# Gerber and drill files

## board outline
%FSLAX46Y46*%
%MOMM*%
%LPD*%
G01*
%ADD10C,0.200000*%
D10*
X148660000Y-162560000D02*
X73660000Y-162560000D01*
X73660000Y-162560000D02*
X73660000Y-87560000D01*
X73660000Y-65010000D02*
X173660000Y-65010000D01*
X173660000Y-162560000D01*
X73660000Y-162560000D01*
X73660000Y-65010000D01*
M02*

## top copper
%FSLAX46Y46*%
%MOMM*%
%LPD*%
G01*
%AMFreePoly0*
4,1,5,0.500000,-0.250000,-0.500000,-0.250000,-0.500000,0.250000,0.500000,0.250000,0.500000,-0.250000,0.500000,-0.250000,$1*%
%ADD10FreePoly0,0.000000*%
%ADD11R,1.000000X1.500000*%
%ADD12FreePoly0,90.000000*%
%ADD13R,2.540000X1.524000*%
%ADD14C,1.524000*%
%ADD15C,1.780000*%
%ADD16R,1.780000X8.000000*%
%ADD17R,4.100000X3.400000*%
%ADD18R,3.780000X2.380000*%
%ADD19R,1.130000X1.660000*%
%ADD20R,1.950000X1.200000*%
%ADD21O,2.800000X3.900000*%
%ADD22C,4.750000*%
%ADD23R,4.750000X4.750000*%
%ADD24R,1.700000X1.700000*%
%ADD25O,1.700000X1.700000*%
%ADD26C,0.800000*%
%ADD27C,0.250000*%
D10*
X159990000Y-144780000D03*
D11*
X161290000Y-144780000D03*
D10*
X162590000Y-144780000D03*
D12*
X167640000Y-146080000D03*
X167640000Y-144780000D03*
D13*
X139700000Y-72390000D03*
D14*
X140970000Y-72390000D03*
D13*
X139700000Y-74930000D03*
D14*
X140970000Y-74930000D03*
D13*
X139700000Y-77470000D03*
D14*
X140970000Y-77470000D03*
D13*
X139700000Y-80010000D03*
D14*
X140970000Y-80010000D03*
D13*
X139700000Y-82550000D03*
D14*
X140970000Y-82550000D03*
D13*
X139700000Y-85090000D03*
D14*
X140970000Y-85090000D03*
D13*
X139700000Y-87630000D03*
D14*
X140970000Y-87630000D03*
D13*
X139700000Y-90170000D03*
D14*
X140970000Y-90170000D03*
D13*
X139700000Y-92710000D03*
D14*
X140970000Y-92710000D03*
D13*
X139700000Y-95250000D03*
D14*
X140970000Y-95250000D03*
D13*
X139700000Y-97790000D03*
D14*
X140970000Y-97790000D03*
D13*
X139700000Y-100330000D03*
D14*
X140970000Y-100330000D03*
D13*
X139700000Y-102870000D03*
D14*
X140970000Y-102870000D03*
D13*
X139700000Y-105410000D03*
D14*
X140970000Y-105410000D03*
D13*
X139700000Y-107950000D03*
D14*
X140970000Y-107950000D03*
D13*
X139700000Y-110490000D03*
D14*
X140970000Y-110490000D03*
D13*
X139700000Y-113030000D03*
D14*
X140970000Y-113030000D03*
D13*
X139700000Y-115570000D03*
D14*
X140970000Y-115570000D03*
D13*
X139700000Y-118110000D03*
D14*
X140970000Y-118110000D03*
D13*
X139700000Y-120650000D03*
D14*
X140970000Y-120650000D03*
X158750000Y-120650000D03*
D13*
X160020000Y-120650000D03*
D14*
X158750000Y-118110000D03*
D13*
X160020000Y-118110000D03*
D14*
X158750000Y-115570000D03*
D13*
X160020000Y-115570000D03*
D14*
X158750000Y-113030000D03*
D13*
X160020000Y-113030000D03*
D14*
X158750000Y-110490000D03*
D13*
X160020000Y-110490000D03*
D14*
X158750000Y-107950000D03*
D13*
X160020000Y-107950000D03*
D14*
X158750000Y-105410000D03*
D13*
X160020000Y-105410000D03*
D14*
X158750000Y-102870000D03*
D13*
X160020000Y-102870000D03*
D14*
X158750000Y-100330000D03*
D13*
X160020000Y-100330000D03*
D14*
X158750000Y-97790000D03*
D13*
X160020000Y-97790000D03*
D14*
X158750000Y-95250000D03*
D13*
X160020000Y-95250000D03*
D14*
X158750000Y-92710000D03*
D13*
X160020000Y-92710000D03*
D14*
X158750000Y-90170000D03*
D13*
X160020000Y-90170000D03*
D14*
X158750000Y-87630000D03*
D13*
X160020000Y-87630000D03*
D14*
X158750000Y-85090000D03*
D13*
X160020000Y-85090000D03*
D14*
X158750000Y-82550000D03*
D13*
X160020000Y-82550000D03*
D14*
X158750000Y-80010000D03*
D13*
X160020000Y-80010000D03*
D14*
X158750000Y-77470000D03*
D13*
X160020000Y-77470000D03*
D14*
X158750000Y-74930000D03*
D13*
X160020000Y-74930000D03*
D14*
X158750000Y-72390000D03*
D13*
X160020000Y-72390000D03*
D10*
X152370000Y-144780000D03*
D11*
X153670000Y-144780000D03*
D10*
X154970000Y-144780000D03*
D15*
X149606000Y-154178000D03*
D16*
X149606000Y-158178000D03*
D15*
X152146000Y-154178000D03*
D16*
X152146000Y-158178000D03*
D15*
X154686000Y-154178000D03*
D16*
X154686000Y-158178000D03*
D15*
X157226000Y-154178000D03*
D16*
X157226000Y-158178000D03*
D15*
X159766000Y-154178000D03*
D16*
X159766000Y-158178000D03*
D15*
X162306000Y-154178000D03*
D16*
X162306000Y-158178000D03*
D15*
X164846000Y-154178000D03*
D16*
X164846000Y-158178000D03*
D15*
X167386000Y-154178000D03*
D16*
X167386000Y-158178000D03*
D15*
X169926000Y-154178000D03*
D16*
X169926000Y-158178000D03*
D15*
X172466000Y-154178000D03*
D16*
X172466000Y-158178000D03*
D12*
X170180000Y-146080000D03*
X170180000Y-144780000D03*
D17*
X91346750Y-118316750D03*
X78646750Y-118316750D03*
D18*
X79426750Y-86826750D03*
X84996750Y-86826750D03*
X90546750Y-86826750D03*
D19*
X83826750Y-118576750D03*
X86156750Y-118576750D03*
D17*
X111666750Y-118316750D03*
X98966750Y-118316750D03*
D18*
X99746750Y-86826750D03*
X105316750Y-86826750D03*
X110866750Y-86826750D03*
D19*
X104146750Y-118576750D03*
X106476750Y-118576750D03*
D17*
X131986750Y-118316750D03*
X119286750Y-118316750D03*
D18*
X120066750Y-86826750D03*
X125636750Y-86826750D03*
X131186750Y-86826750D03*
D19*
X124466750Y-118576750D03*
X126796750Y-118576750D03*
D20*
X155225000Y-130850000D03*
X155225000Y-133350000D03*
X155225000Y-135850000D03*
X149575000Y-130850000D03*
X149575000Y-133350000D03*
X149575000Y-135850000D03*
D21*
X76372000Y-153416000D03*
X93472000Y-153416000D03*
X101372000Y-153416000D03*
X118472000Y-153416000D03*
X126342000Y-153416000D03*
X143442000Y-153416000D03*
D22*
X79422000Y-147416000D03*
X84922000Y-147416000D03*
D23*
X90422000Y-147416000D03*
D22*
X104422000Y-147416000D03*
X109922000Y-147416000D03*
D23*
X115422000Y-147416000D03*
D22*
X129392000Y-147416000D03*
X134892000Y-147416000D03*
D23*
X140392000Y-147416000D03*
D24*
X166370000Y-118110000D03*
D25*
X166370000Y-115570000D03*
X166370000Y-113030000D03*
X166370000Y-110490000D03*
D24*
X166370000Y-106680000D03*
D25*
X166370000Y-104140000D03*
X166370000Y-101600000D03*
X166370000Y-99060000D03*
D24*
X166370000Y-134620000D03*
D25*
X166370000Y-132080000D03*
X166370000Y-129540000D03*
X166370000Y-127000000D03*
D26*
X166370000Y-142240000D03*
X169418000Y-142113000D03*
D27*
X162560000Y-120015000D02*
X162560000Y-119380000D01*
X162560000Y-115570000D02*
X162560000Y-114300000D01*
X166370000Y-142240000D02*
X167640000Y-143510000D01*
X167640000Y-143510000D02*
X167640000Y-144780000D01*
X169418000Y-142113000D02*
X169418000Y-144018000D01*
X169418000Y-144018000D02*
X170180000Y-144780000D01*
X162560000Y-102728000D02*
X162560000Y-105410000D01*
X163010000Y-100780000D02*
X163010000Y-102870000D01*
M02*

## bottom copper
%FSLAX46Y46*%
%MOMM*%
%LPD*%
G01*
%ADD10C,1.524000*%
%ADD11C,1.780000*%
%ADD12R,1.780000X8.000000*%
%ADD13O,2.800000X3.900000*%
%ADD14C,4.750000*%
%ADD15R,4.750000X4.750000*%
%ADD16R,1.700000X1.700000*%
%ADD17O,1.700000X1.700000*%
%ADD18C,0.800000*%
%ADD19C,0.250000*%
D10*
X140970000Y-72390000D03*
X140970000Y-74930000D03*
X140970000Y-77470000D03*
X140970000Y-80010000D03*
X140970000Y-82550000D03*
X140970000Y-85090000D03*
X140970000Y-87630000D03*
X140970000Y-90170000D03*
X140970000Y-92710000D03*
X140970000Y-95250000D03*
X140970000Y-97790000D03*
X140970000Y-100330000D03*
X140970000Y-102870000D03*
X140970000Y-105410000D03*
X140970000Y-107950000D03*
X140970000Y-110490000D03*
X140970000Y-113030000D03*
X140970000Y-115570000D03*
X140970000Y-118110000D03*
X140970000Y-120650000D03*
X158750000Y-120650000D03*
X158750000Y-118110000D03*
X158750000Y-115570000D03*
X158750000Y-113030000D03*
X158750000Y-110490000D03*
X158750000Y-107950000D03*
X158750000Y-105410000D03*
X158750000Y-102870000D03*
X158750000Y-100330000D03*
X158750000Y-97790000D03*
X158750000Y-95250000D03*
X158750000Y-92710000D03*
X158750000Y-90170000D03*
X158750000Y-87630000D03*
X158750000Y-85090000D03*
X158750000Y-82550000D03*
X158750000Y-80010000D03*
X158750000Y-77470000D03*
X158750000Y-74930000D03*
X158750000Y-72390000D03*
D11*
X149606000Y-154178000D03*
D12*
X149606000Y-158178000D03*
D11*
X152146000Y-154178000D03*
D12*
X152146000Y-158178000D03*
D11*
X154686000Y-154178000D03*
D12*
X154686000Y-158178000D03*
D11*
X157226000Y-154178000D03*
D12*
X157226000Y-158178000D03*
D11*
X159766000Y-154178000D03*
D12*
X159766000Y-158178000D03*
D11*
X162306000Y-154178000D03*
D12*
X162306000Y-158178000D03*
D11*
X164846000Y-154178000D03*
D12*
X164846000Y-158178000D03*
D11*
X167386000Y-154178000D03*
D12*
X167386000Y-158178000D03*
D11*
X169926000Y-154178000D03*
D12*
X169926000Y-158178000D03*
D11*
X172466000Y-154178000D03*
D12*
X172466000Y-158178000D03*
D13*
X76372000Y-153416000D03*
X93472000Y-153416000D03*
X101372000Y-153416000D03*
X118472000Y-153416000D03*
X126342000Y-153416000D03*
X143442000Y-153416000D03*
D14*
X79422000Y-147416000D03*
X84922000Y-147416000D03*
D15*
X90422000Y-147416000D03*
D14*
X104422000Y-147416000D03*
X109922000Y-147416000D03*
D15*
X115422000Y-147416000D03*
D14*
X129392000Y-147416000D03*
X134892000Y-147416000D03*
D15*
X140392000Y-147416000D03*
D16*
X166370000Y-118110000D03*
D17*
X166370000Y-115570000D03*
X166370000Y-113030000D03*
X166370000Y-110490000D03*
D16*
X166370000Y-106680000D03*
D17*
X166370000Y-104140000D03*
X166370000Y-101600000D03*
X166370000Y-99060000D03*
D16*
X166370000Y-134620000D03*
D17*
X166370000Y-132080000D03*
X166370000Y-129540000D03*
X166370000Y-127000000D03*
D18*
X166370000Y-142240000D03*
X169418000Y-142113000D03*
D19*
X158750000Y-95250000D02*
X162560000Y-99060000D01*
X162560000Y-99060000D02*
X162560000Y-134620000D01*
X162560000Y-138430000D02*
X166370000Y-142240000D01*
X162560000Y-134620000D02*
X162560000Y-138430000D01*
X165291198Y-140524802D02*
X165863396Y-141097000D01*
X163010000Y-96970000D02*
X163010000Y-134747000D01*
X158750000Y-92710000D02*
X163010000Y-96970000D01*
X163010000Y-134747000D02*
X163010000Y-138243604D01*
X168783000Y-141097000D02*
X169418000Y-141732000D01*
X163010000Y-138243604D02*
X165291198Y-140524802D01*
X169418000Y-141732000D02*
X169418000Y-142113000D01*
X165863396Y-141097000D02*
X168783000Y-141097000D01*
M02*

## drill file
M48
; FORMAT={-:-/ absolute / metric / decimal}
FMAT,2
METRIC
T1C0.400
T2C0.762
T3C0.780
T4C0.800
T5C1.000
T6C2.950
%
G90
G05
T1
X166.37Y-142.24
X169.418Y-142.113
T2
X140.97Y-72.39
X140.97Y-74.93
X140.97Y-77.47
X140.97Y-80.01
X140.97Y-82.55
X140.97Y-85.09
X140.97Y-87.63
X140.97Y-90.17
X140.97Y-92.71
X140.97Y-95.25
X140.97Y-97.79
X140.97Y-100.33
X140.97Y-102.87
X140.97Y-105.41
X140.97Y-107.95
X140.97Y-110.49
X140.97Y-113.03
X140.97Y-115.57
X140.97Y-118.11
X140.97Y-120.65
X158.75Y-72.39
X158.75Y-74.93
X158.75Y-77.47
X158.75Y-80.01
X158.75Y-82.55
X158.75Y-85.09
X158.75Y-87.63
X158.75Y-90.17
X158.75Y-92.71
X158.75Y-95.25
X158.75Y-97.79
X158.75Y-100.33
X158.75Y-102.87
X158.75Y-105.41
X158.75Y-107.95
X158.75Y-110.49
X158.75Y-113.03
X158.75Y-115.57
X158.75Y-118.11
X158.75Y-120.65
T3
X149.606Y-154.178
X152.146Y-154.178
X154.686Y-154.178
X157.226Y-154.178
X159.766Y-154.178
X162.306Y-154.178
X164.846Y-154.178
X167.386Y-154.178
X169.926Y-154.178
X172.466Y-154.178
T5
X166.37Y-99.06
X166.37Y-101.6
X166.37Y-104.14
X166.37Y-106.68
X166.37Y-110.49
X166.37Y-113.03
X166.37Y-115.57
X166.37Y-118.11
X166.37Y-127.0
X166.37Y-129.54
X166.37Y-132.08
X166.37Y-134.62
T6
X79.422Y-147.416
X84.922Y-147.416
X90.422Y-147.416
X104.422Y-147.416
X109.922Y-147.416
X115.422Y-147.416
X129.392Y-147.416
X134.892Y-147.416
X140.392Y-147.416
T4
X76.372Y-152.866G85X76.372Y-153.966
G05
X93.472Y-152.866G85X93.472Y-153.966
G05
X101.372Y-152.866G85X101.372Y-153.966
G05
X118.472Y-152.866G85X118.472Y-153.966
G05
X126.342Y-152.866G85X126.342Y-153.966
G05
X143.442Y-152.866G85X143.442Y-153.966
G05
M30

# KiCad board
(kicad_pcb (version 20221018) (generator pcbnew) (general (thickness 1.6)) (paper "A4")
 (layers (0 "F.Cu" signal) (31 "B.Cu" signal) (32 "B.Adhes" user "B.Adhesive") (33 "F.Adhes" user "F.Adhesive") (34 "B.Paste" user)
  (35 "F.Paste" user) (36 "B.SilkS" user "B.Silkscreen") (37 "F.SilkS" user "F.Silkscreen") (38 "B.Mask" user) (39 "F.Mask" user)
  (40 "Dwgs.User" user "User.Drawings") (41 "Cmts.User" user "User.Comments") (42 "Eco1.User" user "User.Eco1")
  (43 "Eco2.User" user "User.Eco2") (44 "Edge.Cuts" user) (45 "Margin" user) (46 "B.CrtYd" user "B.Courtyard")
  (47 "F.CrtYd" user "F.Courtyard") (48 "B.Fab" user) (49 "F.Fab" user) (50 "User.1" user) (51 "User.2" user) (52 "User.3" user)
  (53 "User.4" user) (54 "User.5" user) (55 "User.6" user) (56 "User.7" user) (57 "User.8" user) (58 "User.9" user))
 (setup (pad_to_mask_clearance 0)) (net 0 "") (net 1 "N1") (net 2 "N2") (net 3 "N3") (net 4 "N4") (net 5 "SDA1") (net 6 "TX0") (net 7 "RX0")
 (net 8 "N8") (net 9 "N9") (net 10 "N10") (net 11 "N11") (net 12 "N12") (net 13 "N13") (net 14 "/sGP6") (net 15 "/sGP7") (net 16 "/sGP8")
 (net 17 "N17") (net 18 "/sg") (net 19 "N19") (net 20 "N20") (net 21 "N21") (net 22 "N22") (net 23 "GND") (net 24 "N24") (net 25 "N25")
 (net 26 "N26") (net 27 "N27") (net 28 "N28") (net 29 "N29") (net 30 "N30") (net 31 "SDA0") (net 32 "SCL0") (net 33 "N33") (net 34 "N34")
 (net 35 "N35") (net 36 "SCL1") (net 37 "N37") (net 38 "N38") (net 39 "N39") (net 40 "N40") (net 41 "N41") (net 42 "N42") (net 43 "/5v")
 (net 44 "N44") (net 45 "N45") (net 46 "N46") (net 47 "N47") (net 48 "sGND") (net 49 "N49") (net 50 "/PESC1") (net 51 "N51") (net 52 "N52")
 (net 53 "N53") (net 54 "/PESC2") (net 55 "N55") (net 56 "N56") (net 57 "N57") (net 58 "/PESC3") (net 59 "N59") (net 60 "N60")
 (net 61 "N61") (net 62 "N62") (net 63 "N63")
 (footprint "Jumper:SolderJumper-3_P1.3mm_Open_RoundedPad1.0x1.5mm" (layer "F.Cu") (at 161.29 144.78)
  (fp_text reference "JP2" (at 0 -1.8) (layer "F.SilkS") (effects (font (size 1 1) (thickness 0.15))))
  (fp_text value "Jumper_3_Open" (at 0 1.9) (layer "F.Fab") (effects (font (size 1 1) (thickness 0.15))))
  (pad "1" smd custom (at -1.3 0) (size 1 0.5) (layers "F.Cu" "F.Mask") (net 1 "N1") (zone_connect 2)
   (options (clearance outline) (anchor rect)) (primitives))
  (pad "2" smd rect (at 0 0) (size 1 1.5) (layers "F.Cu" "F.Mask") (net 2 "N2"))
  (pad "3" smd custom (at 1.3 0) (size 1 0.5) (layers "F.Cu" "F.Mask") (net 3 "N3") (zone_connect 2)
   (options (clearance outline) (anchor rect)) (primitives)))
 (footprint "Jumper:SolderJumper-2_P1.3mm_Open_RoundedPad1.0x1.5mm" (layer "F.Cu") (at 167.64 145.43 90)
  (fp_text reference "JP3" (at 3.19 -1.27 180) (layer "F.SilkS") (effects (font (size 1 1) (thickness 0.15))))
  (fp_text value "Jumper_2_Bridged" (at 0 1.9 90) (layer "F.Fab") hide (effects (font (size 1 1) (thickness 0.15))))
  (pad "1" smd custom (at -0.65 0 90) (size 1 0.5) (layers "F.Cu" "F.Mask") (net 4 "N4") (zone_connect 2)
   (options (clearance outline) (anchor rect)) (primitives))
  (pad "2" smd custom (at 0.65 0 90) (size 1 0.5) (layers "F.Cu" "F.Mask") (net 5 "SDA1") (zone_connect 2)
   (options (clearance outline) (anchor rect)) (primitives)))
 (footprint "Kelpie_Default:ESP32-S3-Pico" (layer "F.Cu") (at 151.13 87.63)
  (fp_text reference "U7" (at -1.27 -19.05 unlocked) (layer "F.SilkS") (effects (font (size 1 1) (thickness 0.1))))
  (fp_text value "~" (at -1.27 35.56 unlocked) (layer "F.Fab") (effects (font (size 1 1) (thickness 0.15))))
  (pad "1" smd rect (at -11.43 -15.24) (size 2.54 1.524) (layers "F.Cu" "B.Adhes" "F.Paste" "F.Mask") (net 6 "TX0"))
  (pad "1" thru_hole circle (at -10.16 -15.24) (size 1.524 1.524) (drill 0.762) (layers "*.Cu" "*.Mask") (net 6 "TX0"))
  (pad "2" smd rect (at -11.43 -12.7) (size 2.54 1.524) (layers "F.Cu" "F.Paste" "F.Mask") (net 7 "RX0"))
  (pad "2" thru_hole circle (at -10.16 -12.7) (size 1.524 1.524) (drill 0.762) (layers "*.Cu" "*.Mask") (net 7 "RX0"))
  (pad "3" smd rect (at -11.43 -10.16) (size 2.54 1.524) (layers "F.Cu" "F.Paste" "F.Mask") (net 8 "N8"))
  (pad "3" thru_hole circle (at -10.16 -10.16) (size 1.524 1.524) (drill 0.762) (layers "*.Cu" "*.Mask") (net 8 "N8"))
  (pad "4" smd rect (at -11.43 -7.62) (size 2.54 1.524) (layers "F.Cu" "F.Paste" "F.Mask") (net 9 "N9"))
  (pad "4" thru_hole circle (at -10.16 -7.62) (size 1.524 1.524) (drill 0.762) (layers "*.Cu" "*.Mask") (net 9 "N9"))
  (pad "5" smd rect (at -11.43 -5.08) (size 2.54 1.524) (layers "F.Cu" "F.Paste" "F.Mask") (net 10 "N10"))
  (pad "5" thru_hole circle (at -10.16 -5.08) (size 1.524 1.524) (drill 0.762) (layers "*.Cu" "*.Mask") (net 10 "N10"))
  (pad "6" smd rect (at -11.43 -2.54) (size 2.54 1.524) (layers "F.Cu" "F.Paste" "F.Mask") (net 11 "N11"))
  (pad "6" thru_hole circle (at -10.16 -2.54) (size 1.524 1.524) (drill 0.762) (layers "*.Cu" "*.Mask") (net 11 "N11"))
  (pad "7" smd rect (at -11.43 0) (size 2.54 1.524) (layers "F.Cu" "F.Paste" "F.Mask") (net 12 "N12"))
  (pad "7" thru_hole circle (at -10.16 0) (size 1.524 1.524) (drill 0.762) (layers "*.Cu" "*.Mask") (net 12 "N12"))
  (pad "8" smd rect (at -11.43 2.54) (size 2.54 1.524) (layers "F.Cu" "F.Paste" "F.Mask") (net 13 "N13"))
  (pad "8" thru_hole circle (at -10.16 2.54) (size 1.524 1.524) (drill 0.762) (layers "*.Cu" "*.Mask") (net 13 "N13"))
  (pad "9" smd rect (at -11.43 5.08) (size 2.54 1.524) (layers "F.Cu" "F.Paste" "F.Mask") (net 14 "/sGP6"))
  (pad "9" thru_hole circle (at -10.16 5.08) (size 1.524 1.524) (drill 0.762) (layers "*.Cu" "*.Mask") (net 14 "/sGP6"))
  (pad "10" smd rect (at -11.43 7.62) (size 2.54 1.524) (layers "F.Cu" "F.Paste" "F.Mask") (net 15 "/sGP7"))
  (pad "10" thru_hole circle (at -10.16 7.62) (size 1.524 1.524) (drill 0.762) (layers "*.Cu" "*.Mask") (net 15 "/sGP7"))
  (pad "11" smd rect (at -11.43 10.16) (size 2.54 1.524) (layers "F.Cu" "F.Paste" "F.Mask") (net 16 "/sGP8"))
  (pad "11" thru_hole circle (at -10.16 10.16) (size 1.524 1.524) (drill 0.762) (layers "*.Cu" "*.Mask") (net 16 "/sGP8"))
  (pad "12" smd rect (at -11.43 12.7) (size 2.54 1.524) (layers "F.Cu" "F.Paste" "F.Mask") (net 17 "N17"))
  (pad "12" thru_hole circle (at -10.16 12.7) (size 1.524 1.524) (drill 0.762) (layers "*.Cu" "*.Mask") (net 17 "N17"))
  (pad "13" smd rect (at -11.43 15.24) (size 2.54 1.524) (layers "F.Cu" "F.Paste" "F.Mask") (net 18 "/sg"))
  (pad "13" thru_hole circle (at -10.16 15.24) (size 1.524 1.524) (drill 0.762) (layers "*.Cu" "*.Mask") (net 18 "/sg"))
  (pad "14" smd rect (at -11.43 17.78) (size 2.54 1.524) (layers "F.Cu" "F.Paste" "F.Mask") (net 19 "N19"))
  (pad "14" thru_hole circle (at -10.16 17.78) (size 1.524 1.524) (drill 0.762) (layers "*.Cu" "*.Mask") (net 19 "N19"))
  (pad "15" smd rect (at -11.43 20.32) (size 2.54 1.524) (layers "F.Cu" "F.Paste" "F.Mask") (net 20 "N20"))
  (pad "15" thru_hole circle (at -10.16 20.32) (size 1.524 1.524) (drill 0.762) (layers "*.Cu" "*.Mask") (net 20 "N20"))
  (pad "16" smd rect (at -11.43 22.86) (size 2.54 1.524) (layers "F.Cu" "F.Paste" "F.Mask") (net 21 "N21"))
  (pad "16" thru_hole circle (at -10.16 22.86) (size 1.524 1.524) (drill 0.762) (layers "*.Cu" "*.Mask") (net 21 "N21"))
  (pad "17" smd rect (at -11.43 25.4) (size 2.54 1.524) (layers "F.Cu" "F.Paste" "F.Mask") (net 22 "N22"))
  (pad "17" thru_hole circle (at -10.16 25.4) (size 1.524 1.524) (drill 0.762) (layers "*.Cu" "*.Mask") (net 22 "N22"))
  (pad "18" smd rect (at -11.43 27.94) (size 2.54 1.524) (layers "F.Cu" "F.Paste" "F.Mask") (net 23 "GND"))
  (pad "18" thru_hole circle (at -10.16 27.94) (size 1.524 1.524) (drill 0.762) (layers "*.Cu" "*.Mask") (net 23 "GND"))
  (pad "19" smd rect (at -11.43 30.48) (size 2.54 1.524) (layers "F.Cu" "F.Paste" "F.Mask") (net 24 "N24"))
  (pad "19" thru_hole circle (at -10.16 30.48) (size 1.524 1.524) (drill 0.762) (layers "*.Cu" "*.Mask") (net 24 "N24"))
  (pad "20" smd rect (at -11.43 33.02) (size 2.54 1.524) (layers "F.Cu" "F.Paste" "F.Mask") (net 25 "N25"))
  (pad "20" thru_hole circle (at -10.16 33.02) (size 1.524 1.524) (drill 0.762) (layers "*.Cu" "*.Mask") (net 25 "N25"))
  (pad "21" thru_hole circle (at 7.62 33.02) (size 1.524 1.524) (drill 0.762) (layers "*.Cu" "*.Mask") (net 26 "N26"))
  (pad "21" smd rect (at 8.89 33.02) (size 2.54 1.524) (layers "F.Cu" "F.Paste" "F.Mask") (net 26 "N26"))
  (pad "22" thru_hole circle (at 7.62 30.48) (size 1.524 1.524) (drill 0.762) (layers "*.Cu" "*.Mask") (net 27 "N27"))
  (pad "22" smd rect (at 8.89 30.48) (size 2.54 1.524) (layers "F.Cu" "F.Paste" "F.Mask") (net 27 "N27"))
  (pad "23" thru_hole circle (at 7.62 27.94) (size 1.524 1.524) (drill 0.762) (layers "*.Cu" "*.Mask") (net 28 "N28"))
  (pad "23" smd rect (at 8.89 27.94) (size 2.54 1.524) (layers "F.Cu" "F.Paste" "F.Mask") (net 28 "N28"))
  (pad "24" thru_hole circle (at 7.62 25.4) (size 1.524 1.524) (drill 0.762) (layers "*.Cu" "*.Mask") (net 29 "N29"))
  (pad "24" smd rect (at 8.89 25.4) (size 2.54 1.524) (layers "F.Cu" "F.Paste" "F.Mask") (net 29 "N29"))
  (pad "25" thru_hole circle (at 7.62 22.86) (size 1.524 1.524) (drill 0.762) (layers "*.Cu" "*.Mask") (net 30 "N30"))
  (pad "25" smd rect (at 8.89 22.86) (size 2.54 1.524) (layers "F.Cu" "F.Paste" "F.Mask") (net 30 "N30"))
  (pad "26" thru_hole circle (at 7.62 20.32) (size 1.524 1.524) (drill 0.762) (layers "*.Cu" "*.Mask") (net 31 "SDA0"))
  (pad "26" smd rect (at 8.89 20.32) (size 2.54 1.524) (layers "F.Cu" "F.Paste" "F.Mask") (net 31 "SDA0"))
  (pad "27" thru_hole circle (at 7.62 17.78) (size 1.524 1.524) (drill 0.762) (layers "*.Cu" "*.Mask") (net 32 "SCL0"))
  (pad "27" smd rect (at 8.89 17.78) (size 2.54 1.524) (layers "F.Cu" "F.Paste" "F.Mask") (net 32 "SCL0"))
  (pad "28" thru_hole circle (at 7.62 15.24) (size 1.524 1.524) (drill 0.762) (layers "*.Cu" "*.Mask") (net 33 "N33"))
  (pad "28" smd rect (at 8.89 15.24) (size 2.54 1.524) (layers "F.Cu" "F.Paste" "F.Mask") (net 33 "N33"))
  (pad "29" thru_hole circle (at 7.62 12.7) (size 1.524 1.524) (drill 0.762) (layers "*.Cu" "*.Mask") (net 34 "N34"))
  (pad "29" smd rect (at 8.89 12.7) (size 2.54 1.524) (layers "F.Cu" "F.Paste" "F.Mask") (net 34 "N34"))
  (pad "30" thru_hole circle (at 7.62 10.16) (size 1.524 1.524) (drill 0.762) (layers "*.Cu" "*.Mask") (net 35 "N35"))
  (pad "30" smd rect (at 8.89 10.16) (size 2.54 1.524) (layers "F.Cu" "F.Paste" "F.Mask") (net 35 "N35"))
  (pad "31" thru_hole circle (at 7.62 7.62) (size 1.524 1.524) (drill 0.762) (layers "*.Cu" "*.Mask") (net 5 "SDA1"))
  (pad "31" smd rect (at 8.89 7.62) (size 2.54 1.524) (layers "F.Cu" "F.Paste" "F.Mask") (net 5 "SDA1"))
  (pad "32" thru_hole circle (at 7.62 5.08) (size 1.524 1.524) (drill 0.762) (layers "*.Cu" "*.Mask") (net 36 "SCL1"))
  (pad "32" smd rect (at 8.89 5.08) (size 2.54 1.524) (layers "F.Cu" "F.Paste" "F.Mask") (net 36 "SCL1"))
  (pad "33" thru_hole circle (at 7.62 2.54) (size 1.524 1.524) (drill 0.762) (layers "*.Cu" "*.Mask") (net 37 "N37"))
  (pad "33" smd rect (at 8.89 2.54) (size 2.54 1.524) (layers "F.Cu" "F.Paste" "F.Mask") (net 37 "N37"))
  (pad "34" thru_hole circle (at 7.62 0) (size 1.524 1.524) (drill 0.762) (layers "*.Cu" "*.Mask") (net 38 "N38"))
  (pad "34" smd rect (at 8.89 0) (size 2.54 1.524) (layers "F.Cu" "F.Paste" "F.Mask") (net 38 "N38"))
  (pad "35" thru_hole circle (at 7.62 -2.54) (size 1.524 1.524) (drill 0.762) (layers "*.Cu" "*.Mask") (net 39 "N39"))
  (pad "35" smd rect (at 8.89 -2.54) (size 2.54 1.524) (layers "F.Cu" "F.Paste" "F.Mask") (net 39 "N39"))
  (pad "36" thru_hole circle (at 7.62 -5.08) (size 1.524 1.524) (drill 0.762) (layers "*.Cu" "*.Mask") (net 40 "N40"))
  (pad "36" smd rect (at 8.89 -5.08) (size 2.54 1.524) (layers "F.Cu" "F.Paste" "F.Mask") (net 40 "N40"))
  (pad "37" thru_hole circle (at 7.62 -7.62) (size 1.524 1.524) (drill 0.762) (layers "*.Cu" "*.Mask") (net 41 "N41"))
  (pad "37" smd rect (at 8.89 -7.62) (size 2.54 1.524) (layers "F.Cu" "F.Paste" "F.Mask") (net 41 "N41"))
  (pad "38" thru_hole circle (at 7.62 -10.16) (size 1.524 1.524) (drill 0.762) (layers "*.Cu" "*.Mask") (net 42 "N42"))
  (pad "38" smd rect (at 8.89 -10.16) (size 2.54 1.524) (layers "F.Cu" "F.Paste" "F.Mask") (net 42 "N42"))
  (pad "39" thru_hole circle (at 7.62 -12.7) (size 1.524 1.524) (drill 0.762) (layers "*.Cu" "*.Mask") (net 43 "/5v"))
  (pad "39" smd rect (at 8.89 -12.7) (size 2.54 1.524) (layers "F.Cu" "F.Paste" "F.Mask") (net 43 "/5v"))
  (pad "40" thru_hole circle (at 7.62 -15.24) (size 1.524 1.524) (drill 0.762) (layers "*.Cu" "*.Mask") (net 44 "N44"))
  (pad "40" smd rect (at 8.89 -15.24) (size 2.54 1.524) (layers "F.Cu" "F.Paste" "F.Mask") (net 44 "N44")))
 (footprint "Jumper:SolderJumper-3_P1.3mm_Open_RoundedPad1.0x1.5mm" (layer "F.Cu") (at 153.67 144.78)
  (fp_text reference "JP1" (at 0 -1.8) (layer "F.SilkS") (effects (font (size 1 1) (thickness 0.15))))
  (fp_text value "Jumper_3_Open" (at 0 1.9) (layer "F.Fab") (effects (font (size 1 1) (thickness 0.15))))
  (pad "1" smd custom (at -1.3 0) (size 1 0.5) (layers "F.Cu" "F.Mask") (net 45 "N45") (zone_connect 2)
   (options (clearance outline) (anchor rect)) (primitives))
  (pad "2" smd rect (at 0 0) (size 1 1.5) (layers "F.Cu" "F.Mask") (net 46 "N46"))
  (pad "3" smd custom (at 1.3 0) (size 1 0.5) (layers "F.Cu" "F.Mask") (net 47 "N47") (zone_connect 2)
   (options (clearance outline) (anchor rect)) (primitives)))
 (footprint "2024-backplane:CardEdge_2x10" (layer "F.Cu") (at 149.606 158.178)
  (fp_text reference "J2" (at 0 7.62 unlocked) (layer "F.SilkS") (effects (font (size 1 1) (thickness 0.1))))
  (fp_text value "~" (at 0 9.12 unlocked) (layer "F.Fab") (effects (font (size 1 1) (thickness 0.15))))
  (pad "1" thru_hole circle (at 0 -4 180) (size 1.78 1.78) (drill 0.78) (layers "*.Cu" "*.Mask") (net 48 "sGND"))
  (pad "1" smd rect (at 0 0 180) (size 1.78 8) (layers "F.Cu" "F.Paste" "F.Mask") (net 48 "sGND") (thermal_bridge_angle 45))
  (pad "1" smd rect (at 0 0) (size 1.78 8) (layers "B.Cu" "B.Paste" "B.Mask") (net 48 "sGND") (thermal_bridge_angle 45))
  (pad "2" thru_hole circle (at 2.54 -4 180) (size 1.78 1.78) (drill 0.78) (layers "*.Cu" "*.Mask") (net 45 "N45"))
  (pad "2" smd rect (at 2.54 0 180) (size 1.78 8) (layers "F.Cu" "F.Paste" "F.Mask") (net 45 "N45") (thermal_bridge_angle 45))
  (pad "2" smd rect (at 2.54 0) (size 1.78 8) (layers "B.Cu" "B.Paste" "B.Mask") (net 45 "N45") (thermal_bridge_angle 45))
  (pad "3" thru_hole circle (at 5.08 -4 180) (size 1.78 1.78) (drill 0.78) (layers "*.Cu" "*.Mask") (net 1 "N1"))
  (pad "3" smd rect (at 5.08 0 180) (size 1.78 8) (layers "F.Cu" "F.Paste" "F.Mask") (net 1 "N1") (thermal_bridge_angle 45))
  (pad "3" smd rect (at 5.08 0) (size 1.78 8) (layers "B.Cu" "B.Paste" "B.Mask") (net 1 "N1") (thermal_bridge_angle 45))
  (pad "4" thru_hole circle (at 7.62 -4 180) (size 1.78 1.78) (drill 0.78) (layers "*.Cu" "*.Mask") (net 48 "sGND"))
  (pad "4" smd rect (at 7.62 0 180) (size 1.78 8) (layers "F.Cu" "F.Paste" "F.Mask") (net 48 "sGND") (thermal_bridge_angle 45))
  (pad "4" smd rect (at 7.62 0) (size 1.78 8) (layers "B.Cu" "B.Paste" "B.Mask") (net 48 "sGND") (thermal_bridge_angle 45))
  (pad "5" thru_hole circle (at 10.16 -4 180) (size 1.78 1.78) (drill 0.78) (layers "*.Cu" "*.Mask") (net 47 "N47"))
  (pad "5" smd rect (at 10.16 0 180) (size 1.78 8) (layers "F.Cu" "F.Paste" "F.Mask") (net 47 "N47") (thermal_bridge_angle 45))
  (pad "5" smd rect (at 10.16 0) (size 1.78 8) (layers "B.Cu" "B.Paste" "B.Mask") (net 47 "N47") (thermal_bridge_angle 45))
  (pad "6" thru_hole circle (at 12.7 -4 180) (size 1.78 1.78) (drill 0.78) (layers "*.Cu" "*.Mask") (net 3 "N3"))
  (pad "6" smd rect (at 12.7 0 180) (size 1.78 8) (layers "F.Cu" "F.Paste" "F.Mask") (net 3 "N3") (thermal_bridge_angle 45))
  (pad "6" smd rect (at 12.7 0) (size 1.78 8) (layers "B.Cu" "B.Paste" "B.Mask") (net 3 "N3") (thermal_bridge_angle 45))
  (pad "7" thru_hole circle (at 15.24 -4 180) (size 1.78 1.78) (drill 0.78) (layers "*.Cu" "*.Mask") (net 48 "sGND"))
  (pad "7" smd rect (at 15.24 0 180) (size 1.78 8) (layers "F.Cu" "F.Paste" "F.Mask") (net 48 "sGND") (thermal_bridge_angle 45))
  (pad "7" smd rect (at 15.24 0) (size 1.78 8) (layers "B.Cu" "B.Paste" "B.Mask") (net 48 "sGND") (thermal_bridge_angle 45))
  (pad "8" thru_hole circle (at 17.78 -4 180) (size 1.78 1.78) (drill 0.78) (layers "*.Cu" "*.Mask") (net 4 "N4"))
  (pad "8" smd rect (at 17.78 0 180) (size 1.78 8) (layers "F.Cu" "F.Paste" "F.Mask") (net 4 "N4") (thermal_bridge_angle 45))
  (pad "8" smd rect (at 17.78 0) (size 1.78 8) (layers "B.Cu" "B.Paste" "B.Mask") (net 4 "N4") (thermal_bridge_angle 45))
  (pad "9" thru_hole circle (at 20.32 -4 180) (size 1.78 1.78) (drill 0.78) (layers "*.Cu" "*.Mask") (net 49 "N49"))
  (pad "9" smd rect (at 20.32 0 180) (size 1.78 8) (layers "F.Cu" "F.Paste" "F.Mask") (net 49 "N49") (thermal_bridge_angle 45))
  (pad "9" smd rect (at 20.32 0) (size 1.78 8) (layers "B.Cu" "B.Paste" "B.Mask") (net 49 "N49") (thermal_bridge_angle 45))
  (pad "10" thru_hole circle (at 22.86 -4 180) (size 1.78 1.78) (drill 0.78) (layers "*.Cu" "*.Mask") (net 48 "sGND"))
  (pad "10" smd rect (at 22.86 0 180) (size 1.78 8) (layers "F.Cu" "F.Paste" "F.Mask") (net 48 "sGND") (thermal_bridge_angle 45))
  (pad "10" smd rect (at 22.86 0) (size 1.78 8) (layers "B.Cu" "B.Paste" "B.Mask") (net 48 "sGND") (thermal_bridge_angle 45)))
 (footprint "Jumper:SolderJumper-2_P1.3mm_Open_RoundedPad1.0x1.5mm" (layer "F.Cu") (at 170.18 145.43 90)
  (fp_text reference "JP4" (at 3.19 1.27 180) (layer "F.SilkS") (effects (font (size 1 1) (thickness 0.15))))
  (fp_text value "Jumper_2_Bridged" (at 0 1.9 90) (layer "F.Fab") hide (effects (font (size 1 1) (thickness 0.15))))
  (pad "1" smd custom (at -0.65 0 90) (size 1 0.5) (layers "F.Cu" "F.Mask") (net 49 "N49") (zone_connect 2)
   (options (clearance outline) (anchor rect)) (primitives))
  (pad "2" smd custom (at 0.65 0 90) (size 1 0.5) (layers "F.Cu" "F.Mask") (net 36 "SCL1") (zone_connect 2)
   (options (clearance outline) (anchor rect)) (primitives)))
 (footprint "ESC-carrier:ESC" (layer "F.Cu") (at 93.39675 120.01675 90)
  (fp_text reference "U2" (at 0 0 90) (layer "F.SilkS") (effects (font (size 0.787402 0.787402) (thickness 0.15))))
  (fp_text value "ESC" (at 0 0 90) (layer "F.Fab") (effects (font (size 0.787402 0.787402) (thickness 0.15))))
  (pad "+" smd rect (at 1.7 -2.05 90) (size 3.4 4.1) (layers "F.Cu" "F.Paste" "F.Mask") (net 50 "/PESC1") (solder_mask_margin 0.102))
  (pad "-" smd rect (at 1.7 -14.75 90) (size 3.4 4.1) (layers "F.Cu" "F.Paste" "F.Mask") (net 23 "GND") (solder_mask_margin 0.102))
  (pad "1" smd rect (at 33.19 -13.97 90) (size 2.38 3.78) (layers "F.Cu" "F.Paste" "F.Mask") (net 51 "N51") (solder_mask_margin 0.102))
  (pad "2" smd rect (at 33.19 -8.4 90) (size 2.38 3.78) (layers "F.Cu" "F.Paste" "F.Mask") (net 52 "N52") (solder_mask_margin 0.102))
  (pad "3" smd rect (at 33.19 -2.85 90) (size 2.38 3.78) (layers "F.Cu" "F.Paste" "F.Mask") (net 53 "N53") (solder_mask_margin 0.102))
  (pad "G" smd rect (at 1.44 -9.57 90) (size 1.66 1.13) (layers "F.Cu" "F.Paste" "F.Mask") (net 18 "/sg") (solder_mask_margin 0.102))
  (pad "S" smd rect (at 1.44 -7.24 90) (size 1.66 1.13) (layers "F.Cu" "F.Paste" "F.Mask") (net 16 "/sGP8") (solder_mask_margin 0.102)))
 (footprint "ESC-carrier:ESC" (layer "F.Cu") (at 113.71675 120.01675 90)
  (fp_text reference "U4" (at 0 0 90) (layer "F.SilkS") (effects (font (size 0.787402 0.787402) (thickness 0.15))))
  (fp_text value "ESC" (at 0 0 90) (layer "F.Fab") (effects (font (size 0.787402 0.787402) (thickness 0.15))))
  (pad "+" smd rect (at 1.7 -2.05 90) (size 3.4 4.1) (layers "F.Cu" "F.Paste" "F.Mask") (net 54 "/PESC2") (solder_mask_margin 0.102))
  (pad "-" smd rect (at 1.7 -14.75 90) (size 3.4 4.1) (layers "F.Cu" "F.Paste" "F.Mask") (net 23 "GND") (solder_mask_margin 0.102))
  (pad "1" smd rect (at 33.19 -13.97 90) (size 2.38 3.78) (layers "F.Cu" "F.Paste" "F.Mask") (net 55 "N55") (solder_mask_margin 0.102))
  (pad "2" smd rect (at 33.19 -8.4 90) (size 2.38 3.78) (layers "F.Cu" "F.Paste" "F.Mask") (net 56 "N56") (solder_mask_margin 0.102))
  (pad "3" smd rect (at 33.19 -2.85 90) (size 2.38 3.78) (layers "F.Cu" "F.Paste" "F.Mask") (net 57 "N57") (solder_mask_margin 0.102))
  (pad "G" smd rect (at 1.44 -9.57 90) (size 1.66 1.13) (layers "F.Cu" "F.Paste" "F.Mask") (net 18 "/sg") (solder_mask_margin 0.102))
  (pad "S" smd rect (at 1.44 -7.24 90) (size 1.66 1.13) (layers "F.Cu" "F.Paste" "F.Mask") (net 15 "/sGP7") (solder_mask_margin 0.102)))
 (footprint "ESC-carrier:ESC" (layer "F.Cu") (at 134.03675 120.01675 90)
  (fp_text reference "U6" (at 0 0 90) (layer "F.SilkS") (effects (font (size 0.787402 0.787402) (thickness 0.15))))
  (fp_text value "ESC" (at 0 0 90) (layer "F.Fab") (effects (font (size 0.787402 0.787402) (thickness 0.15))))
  (pad "+" smd rect (at 1.7 -2.05 90) (size 3.4 4.1) (layers "F.Cu" "F.Paste" "F.Mask") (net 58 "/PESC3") (solder_mask_margin 0.102))
  (pad "-" smd rect (at 1.7 -14.75 90) (size 3.4 4.1) (layers "F.Cu" "F.Paste" "F.Mask") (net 23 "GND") (solder_mask_margin 0.102))
  (pad "1" smd rect (at 33.19 -13.97 90) (size 2.38 3.78) (layers "F.Cu" "F.Paste" "F.Mask") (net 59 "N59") (solder_mask_margin 0.102))
  (pad "2" smd rect (at 33.19 -8.4 90) (size 2.38 3.78) (layers "F.Cu" "F.Paste" "F.Mask") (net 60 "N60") (solder_mask_margin 0.102))
  (pad "3" smd rect (at 33.19 -2.85 90) (size 2.38 3.78) (layers "F.Cu" "F.Paste" "F.Mask") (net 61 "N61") (solder_mask_margin 0.102))
  (pad "G" smd rect (at 1.44 -9.57 90) (size 1.66 1.13) (layers "F.Cu" "F.Paste" "F.Mask") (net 18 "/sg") (solder_mask_margin 0.102))
  (pad "S" smd rect (at 1.44 -7.24 90) (size 1.66 1.13) (layers "F.Cu" "F.Paste" "F.Mask") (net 14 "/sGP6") (solder_mask_margin 0.102)))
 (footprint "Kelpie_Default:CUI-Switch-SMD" (layer "F.Cu") (at 152.4 133.35 -90)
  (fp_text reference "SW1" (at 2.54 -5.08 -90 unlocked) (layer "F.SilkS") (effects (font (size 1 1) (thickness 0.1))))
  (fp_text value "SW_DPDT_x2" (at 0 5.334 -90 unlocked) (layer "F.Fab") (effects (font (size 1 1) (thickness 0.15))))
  (pad "1" smd rect (at -2.5 -2.825 270) (size 1.2 1.95) (layers "F.Cu" "F.Paste" "F.Mask") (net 6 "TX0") (thermal_bridge_angle 45))
  (pad "2" smd rect (at 0 -2.825 270) (size 1.2 1.95) (layers "F.Cu" "F.Paste" "F.Mask") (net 46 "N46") (thermal_bridge_angle 45))
  (pad "3" smd rect (at 2.5 -2.825 270) (size 1.2 1.95) (layers "F.Cu" "F.Paste" "F.Mask") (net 31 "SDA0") (thermal_bridge_angle 45))
  (pad "4" smd rect (at -2.5 2.825 270) (size 1.2 1.95) (layers "F.Cu" "F.Paste" "F.Mask") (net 7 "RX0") (thermal_bridge_angle 45))
  (pad "5" smd rect (at 0 2.825 270) (size 1.2 1.95) (layers "F.Cu" "F.Paste" "F.Mask") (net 2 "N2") (thermal_bridge_angle 45))
  (pad "6" smd rect (at 2.5 2.825 270) (size 1.2 1.95) (layers "F.Cu" "F.Paste" "F.Mask") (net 32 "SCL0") (thermal_bridge_angle 45)))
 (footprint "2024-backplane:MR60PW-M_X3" (layer "F.Cu") (at 109.922 147.416)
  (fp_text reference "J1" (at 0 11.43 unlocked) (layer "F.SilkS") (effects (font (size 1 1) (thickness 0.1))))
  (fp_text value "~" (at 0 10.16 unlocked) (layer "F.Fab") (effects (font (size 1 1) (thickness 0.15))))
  (pad "" thru_hole oval (at -33.55 6) (size 2.8 3.9) (drill oval 0.8 1.9) (layers "*.Cu" "*.Mask"))
  (pad "" thru_hole oval (at -16.45 6) (size 2.8 3.9) (drill oval 0.8 1.9) (layers "*.Cu" "*.Mask"))
  (pad "" thru_hole oval (at -8.55 6) (size 2.8 3.9) (drill oval 0.8 1.9) (layers "*.Cu" "*.Mask"))
  (pad "" thru_hole oval (at 8.55 6) (size 2.8 3.9) (drill oval 0.8 1.9) (layers "*.Cu" "*.Mask"))
  (pad "" thru_hole oval (at 16.42 6) (size 2.8 3.9) (drill oval 0.8 1.9) (layers "*.Cu" "*.Mask"))
  (pad "" thru_hole oval (at 33.52 6) (size 2.8 3.9) (drill oval 0.8 1.9) (layers "*.Cu" "*.Mask"))
  (pad "1" thru_hole circle (at -30.5 0) (size 4.75 4.75) (drill 2.95) (layers "*.Cu" "*.Mask") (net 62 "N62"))
  (pad "2" thru_hole circle (at -25 0) (size 4.75 4.75) (drill 2.95) (layers "*.Cu" "*.Mask") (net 23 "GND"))
  (pad "3" thru_hole rect (at -19.5 0) (size 4.75 4.75) (drill 2.95) (layers "*.Cu" "*.Mask") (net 23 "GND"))
  (pad "4" thru_hole circle (at -5.5 0) (size 4.75 4.75) (drill 2.95) (layers "*.Cu" "*.Mask") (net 50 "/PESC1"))
  (pad "5" thru_hole circle (at 0 0) (size 4.75 4.75) (drill 2.95) (layers "*.Cu" "*.Mask") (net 54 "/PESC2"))
  (pad "6" thru_hole rect (at 5.5 0) (size 4.75 4.75) (drill 2.95) (layers "*.Cu" "*.Mask") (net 58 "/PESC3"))
  (pad "7" thru_hole circle (at 19.47 0) (size 4.75 4.75) (drill 2.95) (layers "*.Cu" "*.Mask") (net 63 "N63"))
  (pad "8" thru_hole circle (at 24.97 0) (size 4.75 4.75) (drill 2.95) (layers "*.Cu" "*.Mask") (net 23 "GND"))
  (pad "9" thru_hole rect (at 30.47 0) (size 4.75 4.75) (drill 2.95) (layers "*.Cu" "*.Mask") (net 43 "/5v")))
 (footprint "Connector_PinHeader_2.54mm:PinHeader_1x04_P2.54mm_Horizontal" (layer "B.Cu") (at 166.37 118.11)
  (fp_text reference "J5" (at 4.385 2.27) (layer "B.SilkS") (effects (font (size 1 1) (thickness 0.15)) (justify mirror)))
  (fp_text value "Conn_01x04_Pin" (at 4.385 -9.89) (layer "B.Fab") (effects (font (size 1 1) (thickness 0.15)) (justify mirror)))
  (pad "1" thru_hole rect (at 0 0) (size 1.7 1.7) (drill 1) (layers "*.Cu" "*.Mask") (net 28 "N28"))
  (pad "2" thru_hole oval (at 0 -2.54) (size 1.7 1.7) (drill 1) (layers "*.Cu" "*.Mask") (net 26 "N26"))
  (pad "3" thru_hole oval (at 0 -5.08) (size 1.7 1.7) (drill 1) (layers "*.Cu" "*.Mask") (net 27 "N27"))
  (pad "4" thru_hole oval (at 0 -7.62) (size 1.7 1.7) (drill 1) (layers "*.Cu" "*.Mask") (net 29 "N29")))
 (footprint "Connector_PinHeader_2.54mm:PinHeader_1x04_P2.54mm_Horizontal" (layer "B.Cu") (at 166.37 106.68)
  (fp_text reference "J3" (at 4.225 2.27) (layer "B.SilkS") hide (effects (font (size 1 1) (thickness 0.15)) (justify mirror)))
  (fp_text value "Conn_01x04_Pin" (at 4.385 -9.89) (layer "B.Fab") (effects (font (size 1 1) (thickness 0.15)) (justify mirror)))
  (pad "1" thru_hole rect (at 0 0) (size 1.7 1.7) (drill 1) (layers "*.Cu" "*.Mask") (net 13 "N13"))
  (pad "2" thru_hole oval (at 0 -2.54) (size 1.7 1.7) (drill 1) (layers "*.Cu" "*.Mask") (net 12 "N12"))
  (pad "3" thru_hole oval (at 0 -5.08) (size 1.7 1.7) (drill 1) (layers "*.Cu" "*.Mask") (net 11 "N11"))
  (pad "4" thru_hole oval (at 0 -7.62) (size 1.7 1.7) (drill 1) (layers "*.Cu" "*.Mask") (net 10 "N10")))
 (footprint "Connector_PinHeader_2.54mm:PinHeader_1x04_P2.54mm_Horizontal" (layer "B.Cu") (at 166.37 134.62)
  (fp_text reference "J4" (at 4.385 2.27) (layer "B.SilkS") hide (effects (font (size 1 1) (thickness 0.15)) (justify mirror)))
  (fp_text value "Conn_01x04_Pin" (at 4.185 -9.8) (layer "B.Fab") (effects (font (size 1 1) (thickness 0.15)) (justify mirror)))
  (pad "1" thru_hole rect (at 0 0) (size 1.7 1.7) (drill 1) (layers "*.Cu" "*.Mask") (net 18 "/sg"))
  (pad "2" thru_hole oval (at 0 -2.54) (size 1.7 1.7) (drill 1) (layers "*.Cu" "*.Mask") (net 14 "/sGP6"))
  (pad "3" thru_hole oval (at 0 -5.08) (size 1.7 1.7) (drill 1) (layers "*.Cu" "*.Mask") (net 15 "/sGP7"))
  (pad "4" thru_hole oval (at 0 -7.62) (size 1.7 1.7) (drill 1) (layers "*.Cu" "*.Mask") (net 16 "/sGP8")))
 (gr_line (start 148.66 162.56) (end 73.66 162.56) (stroke (width 0.2) (type default)) (layer "Edge.Cuts"))
 (gr_line (start 73.66 162.56) (end 73.66 87.56) (stroke (width 0.2) (type default)) (layer "Edge.Cuts"))
 (gr_rect (start 73.66 65.01) (end 173.66 162.56) (stroke (width 0.2) (type default)) (fill none) (layer "Edge.Cuts"))
 (segment (start 162.56 120.015) (end 162.56 119.38) (width 0.25) (layer "F.Cu") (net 26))
 (segment (start 162.56 115.57) (end 162.56 114.3) (width 0.25) (layer "F.Cu") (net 27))
 (segment (start 166.37 142.24) (end 167.64 143.51) (width 0.25) (layer "F.Cu") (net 5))
 (segment (start 167.64 143.51) (end 167.64 144.78) (width 0.25) (layer "F.Cu") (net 5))
 (via (at 166.37 142.24) (size 0.8) (drill 0.4) (layers "F.Cu" "B.Cu") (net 5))
 (segment (start 158.75 95.25) (end 162.56 99.06) (width 0.25) (layer "B.Cu") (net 5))
 (segment (start 162.56 99.06) (end 162.56 134.62) (width 0.25) (layer "B.Cu") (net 5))
 (segment (start 162.56 138.43) (end 166.37 142.24) (width 0.25) (layer "B.Cu") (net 5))
 (segment (start 162.56 134.62) (end 162.56 138.43) (width 0.25) (layer "B.Cu") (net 5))
 (segment (start 169.418 142.113) (end 169.418 144.018) (width 0.25) (layer "F.Cu") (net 36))
 (segment (start 169.418 144.018) (end 170.18 144.78) (width 0.25) (layer "F.Cu") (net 36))
 (via (at 169.418 142.113) (size 0.8) (drill 0.4) (layers "F.Cu" "B.Cu") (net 36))
 (segment (start 165.291198 140.524802) (end 165.863396 141.097) (width 0.25) (layer "B.Cu") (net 36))
 (segment (start 163.01 96.97) (end 163.01 134.747) (width 0.25) (layer "B.Cu") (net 36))
 (segment (start 158.75 92.71) (end 163.01 96.97) (width 0.25) (layer "B.Cu") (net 36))
 (segment (start 163.01 134.747) (end 163.01 138.243604) (width 0.25) (layer "B.Cu") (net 36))
 (segment (start 168.783 141.097) (end 169.418 141.732) (width 0.25) (layer "B.Cu") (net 36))
 (segment (start 163.01 138.243604) (end 165.291198 140.524802) (width 0.25) (layer "B.Cu") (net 36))
 (segment (start 169.418 141.732) (end 169.418 142.113) (width 0.25) (layer "B.Cu") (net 36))
 (segment (start 165.863396 141.097) (end 168.783 141.097) (width 0.25) (layer "B.Cu") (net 36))
 (segment (start 162.56 102.728) (end 162.56 105.41) (width 0.25) (layer "F.Cu") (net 13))
 (segment (start 163.01 100.78) (end 163.01 102.87) (width 0.25) (layer "F.Cu") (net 12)))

